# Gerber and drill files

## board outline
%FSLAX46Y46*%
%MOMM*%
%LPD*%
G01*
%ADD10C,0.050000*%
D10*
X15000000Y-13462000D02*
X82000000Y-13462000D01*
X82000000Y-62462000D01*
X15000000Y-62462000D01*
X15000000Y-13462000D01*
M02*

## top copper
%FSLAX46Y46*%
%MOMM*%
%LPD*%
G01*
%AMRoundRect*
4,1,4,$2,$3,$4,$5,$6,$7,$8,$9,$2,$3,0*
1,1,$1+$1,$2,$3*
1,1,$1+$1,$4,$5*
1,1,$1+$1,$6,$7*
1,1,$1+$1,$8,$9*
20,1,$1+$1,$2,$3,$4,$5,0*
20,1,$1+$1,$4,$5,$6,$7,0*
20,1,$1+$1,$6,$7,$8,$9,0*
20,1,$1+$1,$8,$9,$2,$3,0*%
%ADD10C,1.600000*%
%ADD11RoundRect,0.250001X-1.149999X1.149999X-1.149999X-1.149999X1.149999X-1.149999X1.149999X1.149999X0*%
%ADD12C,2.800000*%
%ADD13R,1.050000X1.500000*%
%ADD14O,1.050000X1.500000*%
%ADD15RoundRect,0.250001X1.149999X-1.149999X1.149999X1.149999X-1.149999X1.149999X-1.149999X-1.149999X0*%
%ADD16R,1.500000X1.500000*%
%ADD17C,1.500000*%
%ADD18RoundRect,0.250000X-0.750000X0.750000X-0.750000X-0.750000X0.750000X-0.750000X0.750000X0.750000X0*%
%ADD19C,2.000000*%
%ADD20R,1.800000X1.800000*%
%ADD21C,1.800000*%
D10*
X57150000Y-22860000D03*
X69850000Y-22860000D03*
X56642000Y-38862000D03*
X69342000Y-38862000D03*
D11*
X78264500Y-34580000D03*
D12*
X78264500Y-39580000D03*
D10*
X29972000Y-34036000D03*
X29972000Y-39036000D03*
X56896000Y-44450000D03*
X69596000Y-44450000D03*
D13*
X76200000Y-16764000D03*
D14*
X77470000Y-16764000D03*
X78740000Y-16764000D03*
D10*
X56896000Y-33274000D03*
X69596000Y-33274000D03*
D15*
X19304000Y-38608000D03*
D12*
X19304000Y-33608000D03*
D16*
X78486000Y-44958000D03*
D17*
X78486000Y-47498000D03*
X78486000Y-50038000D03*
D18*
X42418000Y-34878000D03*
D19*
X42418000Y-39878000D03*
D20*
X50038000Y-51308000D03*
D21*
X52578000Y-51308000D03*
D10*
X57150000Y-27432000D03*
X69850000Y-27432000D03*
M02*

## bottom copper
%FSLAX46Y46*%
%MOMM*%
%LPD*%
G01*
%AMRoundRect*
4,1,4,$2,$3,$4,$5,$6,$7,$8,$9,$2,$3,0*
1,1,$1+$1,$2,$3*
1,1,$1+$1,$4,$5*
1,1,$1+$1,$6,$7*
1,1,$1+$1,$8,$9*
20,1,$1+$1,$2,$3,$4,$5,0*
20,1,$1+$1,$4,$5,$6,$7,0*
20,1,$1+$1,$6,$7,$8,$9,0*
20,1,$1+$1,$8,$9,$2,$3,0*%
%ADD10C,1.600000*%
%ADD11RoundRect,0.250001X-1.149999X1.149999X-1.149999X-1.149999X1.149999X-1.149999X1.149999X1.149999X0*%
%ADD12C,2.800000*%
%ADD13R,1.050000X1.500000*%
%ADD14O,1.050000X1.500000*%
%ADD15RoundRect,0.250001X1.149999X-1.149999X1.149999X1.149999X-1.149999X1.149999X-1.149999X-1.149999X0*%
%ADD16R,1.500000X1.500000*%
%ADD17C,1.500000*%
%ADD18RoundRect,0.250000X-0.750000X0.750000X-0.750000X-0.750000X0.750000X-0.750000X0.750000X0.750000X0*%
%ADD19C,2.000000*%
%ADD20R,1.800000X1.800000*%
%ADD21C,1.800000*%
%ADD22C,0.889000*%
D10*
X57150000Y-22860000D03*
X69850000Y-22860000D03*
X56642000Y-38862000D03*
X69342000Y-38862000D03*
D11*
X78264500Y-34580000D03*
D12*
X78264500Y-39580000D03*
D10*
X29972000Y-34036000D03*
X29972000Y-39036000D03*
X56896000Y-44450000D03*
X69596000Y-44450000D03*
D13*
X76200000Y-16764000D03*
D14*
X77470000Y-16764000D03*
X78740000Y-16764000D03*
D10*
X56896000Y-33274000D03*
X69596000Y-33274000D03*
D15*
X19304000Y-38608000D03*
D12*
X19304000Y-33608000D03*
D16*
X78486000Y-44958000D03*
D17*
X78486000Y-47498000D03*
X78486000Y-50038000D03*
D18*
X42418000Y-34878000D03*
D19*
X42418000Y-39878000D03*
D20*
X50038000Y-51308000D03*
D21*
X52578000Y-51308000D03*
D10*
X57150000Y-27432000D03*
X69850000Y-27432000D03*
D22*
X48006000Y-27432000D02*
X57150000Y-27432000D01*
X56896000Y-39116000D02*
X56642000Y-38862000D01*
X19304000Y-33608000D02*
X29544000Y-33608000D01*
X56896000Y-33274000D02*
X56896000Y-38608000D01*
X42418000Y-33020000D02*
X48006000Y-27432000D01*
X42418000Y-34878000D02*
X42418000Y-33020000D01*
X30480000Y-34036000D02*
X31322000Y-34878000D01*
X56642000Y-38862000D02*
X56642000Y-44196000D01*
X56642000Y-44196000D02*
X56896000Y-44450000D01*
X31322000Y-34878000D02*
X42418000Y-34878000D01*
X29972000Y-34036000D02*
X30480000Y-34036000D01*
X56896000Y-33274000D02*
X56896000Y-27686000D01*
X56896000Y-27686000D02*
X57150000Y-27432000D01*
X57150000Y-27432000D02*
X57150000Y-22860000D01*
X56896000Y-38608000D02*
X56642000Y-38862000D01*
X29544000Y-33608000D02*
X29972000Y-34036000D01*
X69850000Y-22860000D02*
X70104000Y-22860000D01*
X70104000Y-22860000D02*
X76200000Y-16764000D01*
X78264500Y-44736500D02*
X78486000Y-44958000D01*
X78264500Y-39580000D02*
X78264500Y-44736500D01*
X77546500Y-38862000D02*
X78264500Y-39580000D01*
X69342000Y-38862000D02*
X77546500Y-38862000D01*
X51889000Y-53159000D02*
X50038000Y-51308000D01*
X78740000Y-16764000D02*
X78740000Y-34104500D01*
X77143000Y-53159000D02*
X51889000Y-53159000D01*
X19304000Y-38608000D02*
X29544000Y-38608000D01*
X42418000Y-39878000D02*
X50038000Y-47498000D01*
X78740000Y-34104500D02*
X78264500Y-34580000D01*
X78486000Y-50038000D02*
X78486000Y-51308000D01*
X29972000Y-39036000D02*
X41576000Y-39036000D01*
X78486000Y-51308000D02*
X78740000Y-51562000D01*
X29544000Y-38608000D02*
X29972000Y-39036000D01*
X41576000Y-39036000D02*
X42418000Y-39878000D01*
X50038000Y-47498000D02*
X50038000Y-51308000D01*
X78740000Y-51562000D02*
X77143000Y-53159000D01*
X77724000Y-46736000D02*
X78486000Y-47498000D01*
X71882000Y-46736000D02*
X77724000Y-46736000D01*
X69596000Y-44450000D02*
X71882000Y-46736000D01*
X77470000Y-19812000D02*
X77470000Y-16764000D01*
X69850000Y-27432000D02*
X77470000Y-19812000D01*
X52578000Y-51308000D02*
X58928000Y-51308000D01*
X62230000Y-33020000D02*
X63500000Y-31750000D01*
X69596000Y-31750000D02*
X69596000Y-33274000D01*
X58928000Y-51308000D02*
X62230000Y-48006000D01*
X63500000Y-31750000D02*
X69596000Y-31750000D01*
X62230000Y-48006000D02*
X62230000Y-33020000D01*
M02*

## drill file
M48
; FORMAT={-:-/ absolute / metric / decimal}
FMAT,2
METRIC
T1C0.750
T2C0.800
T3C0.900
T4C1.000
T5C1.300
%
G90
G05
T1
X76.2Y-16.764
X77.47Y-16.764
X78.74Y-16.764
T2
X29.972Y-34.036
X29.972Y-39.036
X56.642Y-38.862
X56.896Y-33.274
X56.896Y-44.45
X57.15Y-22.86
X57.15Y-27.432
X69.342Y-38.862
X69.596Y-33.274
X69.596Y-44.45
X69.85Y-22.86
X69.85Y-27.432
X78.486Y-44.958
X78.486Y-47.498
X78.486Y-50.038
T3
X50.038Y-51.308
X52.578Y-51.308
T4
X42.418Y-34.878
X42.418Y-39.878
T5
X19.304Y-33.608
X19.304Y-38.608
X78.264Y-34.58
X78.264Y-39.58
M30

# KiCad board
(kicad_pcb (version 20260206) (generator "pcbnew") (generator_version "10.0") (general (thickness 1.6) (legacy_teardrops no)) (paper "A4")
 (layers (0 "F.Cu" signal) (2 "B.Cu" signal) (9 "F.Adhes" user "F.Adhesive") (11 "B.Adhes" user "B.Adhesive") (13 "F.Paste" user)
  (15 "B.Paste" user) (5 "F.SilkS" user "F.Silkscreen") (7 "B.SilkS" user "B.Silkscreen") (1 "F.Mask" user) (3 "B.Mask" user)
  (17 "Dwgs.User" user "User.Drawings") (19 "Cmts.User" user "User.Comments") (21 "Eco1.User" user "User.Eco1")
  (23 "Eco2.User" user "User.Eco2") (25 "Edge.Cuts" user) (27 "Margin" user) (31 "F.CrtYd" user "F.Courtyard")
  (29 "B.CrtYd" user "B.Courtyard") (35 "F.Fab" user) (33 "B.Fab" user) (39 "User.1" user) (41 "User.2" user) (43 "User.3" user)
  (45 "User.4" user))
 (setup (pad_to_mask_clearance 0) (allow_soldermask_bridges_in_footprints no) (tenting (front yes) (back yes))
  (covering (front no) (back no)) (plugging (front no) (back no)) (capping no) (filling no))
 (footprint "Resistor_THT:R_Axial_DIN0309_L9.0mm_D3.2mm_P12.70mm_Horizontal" (layer "F.Cu") (at 57.15 22.86)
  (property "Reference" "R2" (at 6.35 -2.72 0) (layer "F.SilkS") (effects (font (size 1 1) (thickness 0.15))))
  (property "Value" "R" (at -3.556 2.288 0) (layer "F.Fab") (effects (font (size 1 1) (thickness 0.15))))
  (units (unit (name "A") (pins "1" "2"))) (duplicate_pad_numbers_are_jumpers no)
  (pad "1" thru_hole circle (at 0 0) (size 1.6 1.6) (drill 0.8) (layers "*.Cu" "*.Mask") (remove_unused_layers no) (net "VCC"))
  (pad "2" thru_hole circle (at 12.7 0) (size 1.6 1.6) (drill 0.8) (layers "*.Cu" "*.Mask") (remove_unused_layers no) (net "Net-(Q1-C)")))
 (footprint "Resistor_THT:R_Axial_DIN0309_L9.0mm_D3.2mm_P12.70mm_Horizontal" (layer "F.Cu") (at 56.642 38.862)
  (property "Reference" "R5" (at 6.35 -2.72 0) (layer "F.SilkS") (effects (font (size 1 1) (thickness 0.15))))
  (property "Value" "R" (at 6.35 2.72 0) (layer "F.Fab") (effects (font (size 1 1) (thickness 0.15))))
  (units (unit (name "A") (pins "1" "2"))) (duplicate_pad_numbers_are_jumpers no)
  (pad "1" thru_hole circle (at 0 0) (size 1.6 1.6) (drill 0.8) (layers "*.Cu" "*.Mask") (remove_unused_layers no) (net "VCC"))
  (pad "2" thru_hole circle (at 12.7 0) (size 1.6 1.6) (drill 0.8) (layers "*.Cu" "*.Mask") (remove_unused_layers no) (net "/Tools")))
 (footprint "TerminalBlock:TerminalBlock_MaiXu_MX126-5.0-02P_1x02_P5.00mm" (layer "F.Cu") (at 78.2645 34.58 -90)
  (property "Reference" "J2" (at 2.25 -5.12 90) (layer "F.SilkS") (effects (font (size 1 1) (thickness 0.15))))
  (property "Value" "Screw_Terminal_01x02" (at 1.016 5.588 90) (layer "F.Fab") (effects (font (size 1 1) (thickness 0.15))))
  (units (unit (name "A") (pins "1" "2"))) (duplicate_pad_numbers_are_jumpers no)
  (pad "1" thru_hole roundrect (at 0 0 270) (size 2.8 2.8) (drill 1.3) (layers "*.Cu" "*.Mask") (remove_unused_layers no)
   (roundrect_rratio 0.089286) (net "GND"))
  (pad "2" thru_hole circle (at 5 0 270) (size 2.8 2.8) (drill 1.3) (layers "*.Cu" "*.Mask") (remove_unused_layers no) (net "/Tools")))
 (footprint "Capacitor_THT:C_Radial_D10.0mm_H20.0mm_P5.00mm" (layer "F.Cu") (at 29.972 34.036 -90)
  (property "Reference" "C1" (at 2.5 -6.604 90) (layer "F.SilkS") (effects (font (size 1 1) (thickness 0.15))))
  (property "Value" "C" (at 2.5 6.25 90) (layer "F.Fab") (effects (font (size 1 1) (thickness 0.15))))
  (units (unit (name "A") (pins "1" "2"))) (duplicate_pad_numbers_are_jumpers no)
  (pad "1" thru_hole circle (at 0 0 270) (size 1.6 1.6) (drill 0.8) (layers "*.Cu" "*.Mask") (remove_unused_layers no) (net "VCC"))
  (pad "2" thru_hole circle (at 5 0 270) (size 1.6 1.6) (drill 0.8) (layers "*.Cu" "*.Mask") (remove_unused_layers no) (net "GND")))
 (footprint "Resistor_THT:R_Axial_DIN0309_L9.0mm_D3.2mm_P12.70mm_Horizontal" (layer "F.Cu") (at 56.896 44.45)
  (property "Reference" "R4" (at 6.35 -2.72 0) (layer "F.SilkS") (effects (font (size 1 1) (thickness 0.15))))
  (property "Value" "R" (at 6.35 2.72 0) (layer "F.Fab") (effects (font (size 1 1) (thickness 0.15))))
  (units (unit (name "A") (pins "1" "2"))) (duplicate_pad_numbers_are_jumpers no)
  (pad "1" thru_hole circle (at 0 0) (size 1.6 1.6) (drill 0.8) (layers "*.Cu" "*.Mask") (remove_unused_layers no) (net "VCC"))
  (pad "2" thru_hole circle (at 12.7 0) (size 1.6 1.6) (drill 0.8) (layers "*.Cu" "*.Mask") (remove_unused_layers no) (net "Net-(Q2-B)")))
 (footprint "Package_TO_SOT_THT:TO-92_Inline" (layer "F.Cu") (at 76.2 16.764)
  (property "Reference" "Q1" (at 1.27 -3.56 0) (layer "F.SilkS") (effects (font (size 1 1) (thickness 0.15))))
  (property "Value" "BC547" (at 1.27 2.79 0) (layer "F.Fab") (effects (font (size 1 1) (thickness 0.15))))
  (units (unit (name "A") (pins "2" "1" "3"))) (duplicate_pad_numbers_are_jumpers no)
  (pad "1" thru_hole rect (at 0 0) (size 1.05 1.5) (drill 0.75) (layers "*.Cu" "*.Mask") (remove_unused_layers no) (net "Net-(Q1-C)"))
  (pad "2" thru_hole oval (at 1.27 0) (size 1.05 1.5) (drill 0.75) (layers "*.Cu" "*.Mask") (remove_unused_layers no) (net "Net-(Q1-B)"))
  (pad "3" thru_hole oval (at 2.54 0) (size 1.05 1.5) (drill 0.75) (layers "*.Cu" "*.Mask") (remove_unused_layers no) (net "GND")))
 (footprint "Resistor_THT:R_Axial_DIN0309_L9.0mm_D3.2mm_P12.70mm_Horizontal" (layer "F.Cu") (at 56.896 33.274)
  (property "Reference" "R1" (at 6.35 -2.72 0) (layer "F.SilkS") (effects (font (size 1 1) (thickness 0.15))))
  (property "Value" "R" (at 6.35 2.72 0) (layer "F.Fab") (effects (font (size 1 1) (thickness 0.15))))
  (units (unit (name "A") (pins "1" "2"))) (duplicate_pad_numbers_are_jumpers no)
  (pad "1" thru_hole circle (at 0 0) (size 1.6 1.6) (drill 0.8) (layers "*.Cu" "*.Mask") (remove_unused_layers no) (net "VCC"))
  (pad "2" thru_hole circle (at 12.7 0) (size 1.6 1.6) (drill 0.8) (layers "*.Cu" "*.Mask") (remove_unused_layers no) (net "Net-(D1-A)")))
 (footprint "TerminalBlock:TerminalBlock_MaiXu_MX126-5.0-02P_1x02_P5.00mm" (layer "F.Cu") (at 19.304 38.608 90)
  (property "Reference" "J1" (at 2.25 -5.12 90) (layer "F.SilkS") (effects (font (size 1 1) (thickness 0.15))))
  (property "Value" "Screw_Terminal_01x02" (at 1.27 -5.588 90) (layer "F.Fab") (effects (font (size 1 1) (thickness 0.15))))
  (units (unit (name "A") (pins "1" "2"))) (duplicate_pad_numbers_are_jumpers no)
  (pad "1" thru_hole roundrect (at 0 0 90) (size 2.8 2.8) (drill 1.3) (layers "*.Cu" "*.Mask") (remove_unused_layers no)
   (roundrect_rratio 0.089286) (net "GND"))
  (pad "2" thru_hole circle (at 5 0 90) (size 2.8 2.8) (drill 1.3) (layers "*.Cu" "*.Mask") (remove_unused_layers no) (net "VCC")))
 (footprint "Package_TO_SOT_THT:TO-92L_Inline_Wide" (layer "F.Cu") (at 78.486 44.958 -90)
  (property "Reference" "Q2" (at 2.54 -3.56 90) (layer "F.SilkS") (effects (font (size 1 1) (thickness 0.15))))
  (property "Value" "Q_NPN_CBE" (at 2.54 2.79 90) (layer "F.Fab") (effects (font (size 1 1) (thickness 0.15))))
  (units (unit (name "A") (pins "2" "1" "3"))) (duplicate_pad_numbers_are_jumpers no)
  (pad "1" thru_hole rect (at 0 0 270) (size 1.5 1.5) (drill 0.8) (layers "*.Cu" "*.Mask") (remove_unused_layers no) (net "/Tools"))
  (pad "2" thru_hole circle (at 2.54 0 270) (size 1.5 1.5) (drill 0.8) (layers "*.Cu" "*.Mask") (remove_unused_layers no) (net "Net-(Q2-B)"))
  (pad "3" thru_hole circle (at 5.08 0 270) (size 1.5 1.5) (drill 0.8) (layers "*.Cu" "*.Mask") (remove_unused_layers no) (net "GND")))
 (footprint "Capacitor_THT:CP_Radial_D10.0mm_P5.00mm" (layer "F.Cu") (at 42.418 34.878 -90)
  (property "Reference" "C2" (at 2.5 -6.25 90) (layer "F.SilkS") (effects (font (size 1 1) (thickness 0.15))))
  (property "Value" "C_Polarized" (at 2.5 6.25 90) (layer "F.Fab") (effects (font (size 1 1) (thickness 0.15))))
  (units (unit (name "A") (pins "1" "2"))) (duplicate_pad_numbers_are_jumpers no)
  (pad "1" thru_hole roundrect (at 0 0 270) (size 2 2) (drill 1) (layers "*.Cu" "*.Mask") (remove_unused_layers no) (roundrect_rratio 0.125)
   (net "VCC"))
  (pad "2" thru_hole circle (at 5 0 270) (size 2 2) (drill 1) (layers "*.Cu" "*.Mask") (remove_unused_layers no) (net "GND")))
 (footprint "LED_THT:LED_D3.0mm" (layer "F.Cu") (at 50.038 51.308)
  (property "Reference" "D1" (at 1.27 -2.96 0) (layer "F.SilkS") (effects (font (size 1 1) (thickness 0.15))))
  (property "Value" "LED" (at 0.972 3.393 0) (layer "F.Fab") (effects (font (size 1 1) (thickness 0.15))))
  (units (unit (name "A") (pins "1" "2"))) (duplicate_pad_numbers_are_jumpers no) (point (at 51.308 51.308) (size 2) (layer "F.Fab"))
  (pad "1" thru_hole rect (at 0 0) (size 1.8 1.8) (drill 0.9) (layers "*.Cu" "*.Mask") (remove_unused_layers no) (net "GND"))
  (pad "2" thru_hole circle (at 2.54 0) (size 1.8 1.8) (drill 0.9) (layers "*.Cu" "*.Mask") (remove_unused_layers no) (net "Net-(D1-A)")))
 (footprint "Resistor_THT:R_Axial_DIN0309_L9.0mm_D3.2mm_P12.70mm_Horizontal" (layer "F.Cu") (at 57.15 27.432)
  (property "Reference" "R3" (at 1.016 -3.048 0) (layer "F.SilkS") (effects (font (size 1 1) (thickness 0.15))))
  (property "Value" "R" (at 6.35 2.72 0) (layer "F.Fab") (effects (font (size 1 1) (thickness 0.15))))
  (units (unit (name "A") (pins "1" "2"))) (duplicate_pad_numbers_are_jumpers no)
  (pad "1" thru_hole circle (at 0 0) (size 1.6 1.6) (drill 0.8) (layers "*.Cu" "*.Mask") (remove_unused_layers no) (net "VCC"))
  (pad "2" thru_hole circle (at 12.7 0) (size 1.6 1.6) (drill 0.8) (layers "*.Cu" "*.Mask") (remove_unused_layers no) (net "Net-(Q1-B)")))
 (gr_rect (start 15 13.462) (end 82 62.462) (stroke (width 0.05) (type default)) (fill no) (layer "Edge.Cuts"))
 (segment (start 48.006 27.432) (end 57.15 27.432) (width 0.889) (layer "B.Cu") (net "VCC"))
 (segment (start 56.896 39.116) (end 56.642 38.862) (width 0.889) (layer "B.Cu") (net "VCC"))
 (segment (start 19.304 33.608) (end 29.544 33.608) (width 0.889) (layer "B.Cu") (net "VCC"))
 (segment (start 56.896 33.274) (end 56.896 38.608) (width 0.889) (layer "B.Cu") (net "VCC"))
 (segment (start 42.418 33.02) (end 48.006 27.432) (width 0.889) (layer "B.Cu") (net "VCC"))
 (segment (start 42.418 34.878) (end 42.418 33.02) (width 0.889) (layer "B.Cu") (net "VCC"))
 (segment (start 30.48 34.036) (end 31.322 34.878) (width 0.889) (layer "B.Cu") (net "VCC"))
 (segment (start 56.642 38.862) (end 56.642 44.196) (width 0.889) (layer "B.Cu") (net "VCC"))
 (segment (start 56.642 44.196) (end 56.896 44.45) (width 0.889) (layer "B.Cu") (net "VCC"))
 (segment (start 31.322 34.878) (end 42.418 34.878) (width 0.889) (layer "B.Cu") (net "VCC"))
 (segment (start 29.972 34.036) (end 30.48 34.036) (width 0.889) (layer "B.Cu") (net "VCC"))
 (segment (start 56.896 33.274) (end 56.896 27.686) (width 0.889) (layer "B.Cu") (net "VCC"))
 (segment (start 56.896 27.686) (end 57.15 27.432) (width 0.889) (layer "B.Cu") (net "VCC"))
 (segment (start 57.15 27.432) (end 57.15 22.86) (width 0.889) (layer "B.Cu") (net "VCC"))
 (segment (start 56.896 38.608) (end 56.642 38.862) (width 0.889) (layer "B.Cu") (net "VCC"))
 (segment (start 29.544 33.608) (end 29.972 34.036) (width 0.889) (layer "B.Cu") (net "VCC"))
 (segment (start 69.85 22.86) (end 70.104 22.86) (width 0.889) (layer "B.Cu") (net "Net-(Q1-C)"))
 (segment (start 70.104 22.86) (end 76.2 16.764) (width 0.889) (layer "B.Cu") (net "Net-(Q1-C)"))
 (segment (start 78.2645 44.7365) (end 78.486 44.958) (width 0.889) (layer "B.Cu") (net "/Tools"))
 (segment (start 78.2645 39.58) (end 78.2645 44.7365) (width 0.889) (layer "B.Cu") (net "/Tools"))
 (segment (start 77.5465 38.862) (end 78.2645 39.58) (width 0.889) (layer "B.Cu") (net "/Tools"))
 (segment (start 69.342 38.862) (end 77.5465 38.862) (width 0.889) (layer "B.Cu") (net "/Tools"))
 (segment (start 51.889 53.159) (end 50.038 51.308) (width 0.889) (layer "B.Cu") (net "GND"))
 (segment (start 78.74 16.764) (end 78.74 34.1045) (width 0.889) (layer "B.Cu") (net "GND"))
 (segment (start 77.143 53.159) (end 51.889 53.159) (width 0.889) (layer "B.Cu") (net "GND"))
 (segment (start 19.304 38.608) (end 29.544 38.608) (width 0.889) (layer "B.Cu") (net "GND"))
 (segment (start 42.418 39.878) (end 50.038 47.498) (width 0.889) (layer "B.Cu") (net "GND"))
 (segment (start 78.74 34.1045) (end 78.2645 34.58) (width 0.889) (layer "B.Cu") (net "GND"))
 (segment (start 78.486 50.038) (end 78.486 51.308) (width 0.889) (layer "B.Cu") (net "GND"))
 (segment (start 29.972 39.036) (end 41.576 39.036) (width 0.889) (layer "B.Cu") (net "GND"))
 (segment (start 78.486 51.308) (end 78.74 51.562) (width 0.889) (layer "B.Cu") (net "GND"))
 (segment (start 29.544 38.608) (end 29.972 39.036) (width 0.889) (layer "B.Cu") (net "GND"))
 (segment (start 41.576 39.036) (end 42.418 39.878) (width 0.889) (layer "B.Cu") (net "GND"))
 (segment (start 50.038 47.498) (end 50.038 51.308) (width 0.889) (layer "B.Cu") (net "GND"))
 (segment (start 78.74 51.562) (end 77.143 53.159) (width 0.889) (layer "B.Cu") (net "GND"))
 (segment (start 77.724 46.736) (end 78.486 47.498) (width 0.889) (layer "B.Cu") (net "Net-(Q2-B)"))
 (segment (start 71.882 46.736) (end 77.724 46.736) (width 0.889) (layer "B.Cu") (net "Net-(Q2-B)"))
 (segment (start 69.596 44.45) (end 71.882 46.736) (width 0.889) (layer "B.Cu") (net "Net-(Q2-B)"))
 (segment (start 77.47 19.812) (end 77.47 16.764) (width 0.889) (layer "B.Cu") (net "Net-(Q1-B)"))
 (segment (start 69.85 27.432) (end 77.47 19.812) (width 0.889) (layer "B.Cu") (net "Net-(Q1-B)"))
 (segment (start 52.578 51.308) (end 58.928 51.308) (width 0.889) (layer "B.Cu") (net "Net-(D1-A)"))
 (segment (start 62.23 33.02) (end 63.5 31.75) (width 0.889) (layer "B.Cu") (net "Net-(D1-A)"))
 (segment (start 69.596 31.75) (end 69.596 33.274) (width 0.889) (layer "B.Cu") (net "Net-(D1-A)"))
 (segment (start 58.928 51.308) (end 62.23 48.006) (width 0.889) (layer "B.Cu") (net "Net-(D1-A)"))
 (segment (start 63.5 31.75) (end 69.596 31.75) (width 0.889) (layer "B.Cu") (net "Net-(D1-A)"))
 (segment (start 62.23 48.006) (end 62.23 33.02) (width 0.889) (layer "B.Cu") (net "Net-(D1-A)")))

